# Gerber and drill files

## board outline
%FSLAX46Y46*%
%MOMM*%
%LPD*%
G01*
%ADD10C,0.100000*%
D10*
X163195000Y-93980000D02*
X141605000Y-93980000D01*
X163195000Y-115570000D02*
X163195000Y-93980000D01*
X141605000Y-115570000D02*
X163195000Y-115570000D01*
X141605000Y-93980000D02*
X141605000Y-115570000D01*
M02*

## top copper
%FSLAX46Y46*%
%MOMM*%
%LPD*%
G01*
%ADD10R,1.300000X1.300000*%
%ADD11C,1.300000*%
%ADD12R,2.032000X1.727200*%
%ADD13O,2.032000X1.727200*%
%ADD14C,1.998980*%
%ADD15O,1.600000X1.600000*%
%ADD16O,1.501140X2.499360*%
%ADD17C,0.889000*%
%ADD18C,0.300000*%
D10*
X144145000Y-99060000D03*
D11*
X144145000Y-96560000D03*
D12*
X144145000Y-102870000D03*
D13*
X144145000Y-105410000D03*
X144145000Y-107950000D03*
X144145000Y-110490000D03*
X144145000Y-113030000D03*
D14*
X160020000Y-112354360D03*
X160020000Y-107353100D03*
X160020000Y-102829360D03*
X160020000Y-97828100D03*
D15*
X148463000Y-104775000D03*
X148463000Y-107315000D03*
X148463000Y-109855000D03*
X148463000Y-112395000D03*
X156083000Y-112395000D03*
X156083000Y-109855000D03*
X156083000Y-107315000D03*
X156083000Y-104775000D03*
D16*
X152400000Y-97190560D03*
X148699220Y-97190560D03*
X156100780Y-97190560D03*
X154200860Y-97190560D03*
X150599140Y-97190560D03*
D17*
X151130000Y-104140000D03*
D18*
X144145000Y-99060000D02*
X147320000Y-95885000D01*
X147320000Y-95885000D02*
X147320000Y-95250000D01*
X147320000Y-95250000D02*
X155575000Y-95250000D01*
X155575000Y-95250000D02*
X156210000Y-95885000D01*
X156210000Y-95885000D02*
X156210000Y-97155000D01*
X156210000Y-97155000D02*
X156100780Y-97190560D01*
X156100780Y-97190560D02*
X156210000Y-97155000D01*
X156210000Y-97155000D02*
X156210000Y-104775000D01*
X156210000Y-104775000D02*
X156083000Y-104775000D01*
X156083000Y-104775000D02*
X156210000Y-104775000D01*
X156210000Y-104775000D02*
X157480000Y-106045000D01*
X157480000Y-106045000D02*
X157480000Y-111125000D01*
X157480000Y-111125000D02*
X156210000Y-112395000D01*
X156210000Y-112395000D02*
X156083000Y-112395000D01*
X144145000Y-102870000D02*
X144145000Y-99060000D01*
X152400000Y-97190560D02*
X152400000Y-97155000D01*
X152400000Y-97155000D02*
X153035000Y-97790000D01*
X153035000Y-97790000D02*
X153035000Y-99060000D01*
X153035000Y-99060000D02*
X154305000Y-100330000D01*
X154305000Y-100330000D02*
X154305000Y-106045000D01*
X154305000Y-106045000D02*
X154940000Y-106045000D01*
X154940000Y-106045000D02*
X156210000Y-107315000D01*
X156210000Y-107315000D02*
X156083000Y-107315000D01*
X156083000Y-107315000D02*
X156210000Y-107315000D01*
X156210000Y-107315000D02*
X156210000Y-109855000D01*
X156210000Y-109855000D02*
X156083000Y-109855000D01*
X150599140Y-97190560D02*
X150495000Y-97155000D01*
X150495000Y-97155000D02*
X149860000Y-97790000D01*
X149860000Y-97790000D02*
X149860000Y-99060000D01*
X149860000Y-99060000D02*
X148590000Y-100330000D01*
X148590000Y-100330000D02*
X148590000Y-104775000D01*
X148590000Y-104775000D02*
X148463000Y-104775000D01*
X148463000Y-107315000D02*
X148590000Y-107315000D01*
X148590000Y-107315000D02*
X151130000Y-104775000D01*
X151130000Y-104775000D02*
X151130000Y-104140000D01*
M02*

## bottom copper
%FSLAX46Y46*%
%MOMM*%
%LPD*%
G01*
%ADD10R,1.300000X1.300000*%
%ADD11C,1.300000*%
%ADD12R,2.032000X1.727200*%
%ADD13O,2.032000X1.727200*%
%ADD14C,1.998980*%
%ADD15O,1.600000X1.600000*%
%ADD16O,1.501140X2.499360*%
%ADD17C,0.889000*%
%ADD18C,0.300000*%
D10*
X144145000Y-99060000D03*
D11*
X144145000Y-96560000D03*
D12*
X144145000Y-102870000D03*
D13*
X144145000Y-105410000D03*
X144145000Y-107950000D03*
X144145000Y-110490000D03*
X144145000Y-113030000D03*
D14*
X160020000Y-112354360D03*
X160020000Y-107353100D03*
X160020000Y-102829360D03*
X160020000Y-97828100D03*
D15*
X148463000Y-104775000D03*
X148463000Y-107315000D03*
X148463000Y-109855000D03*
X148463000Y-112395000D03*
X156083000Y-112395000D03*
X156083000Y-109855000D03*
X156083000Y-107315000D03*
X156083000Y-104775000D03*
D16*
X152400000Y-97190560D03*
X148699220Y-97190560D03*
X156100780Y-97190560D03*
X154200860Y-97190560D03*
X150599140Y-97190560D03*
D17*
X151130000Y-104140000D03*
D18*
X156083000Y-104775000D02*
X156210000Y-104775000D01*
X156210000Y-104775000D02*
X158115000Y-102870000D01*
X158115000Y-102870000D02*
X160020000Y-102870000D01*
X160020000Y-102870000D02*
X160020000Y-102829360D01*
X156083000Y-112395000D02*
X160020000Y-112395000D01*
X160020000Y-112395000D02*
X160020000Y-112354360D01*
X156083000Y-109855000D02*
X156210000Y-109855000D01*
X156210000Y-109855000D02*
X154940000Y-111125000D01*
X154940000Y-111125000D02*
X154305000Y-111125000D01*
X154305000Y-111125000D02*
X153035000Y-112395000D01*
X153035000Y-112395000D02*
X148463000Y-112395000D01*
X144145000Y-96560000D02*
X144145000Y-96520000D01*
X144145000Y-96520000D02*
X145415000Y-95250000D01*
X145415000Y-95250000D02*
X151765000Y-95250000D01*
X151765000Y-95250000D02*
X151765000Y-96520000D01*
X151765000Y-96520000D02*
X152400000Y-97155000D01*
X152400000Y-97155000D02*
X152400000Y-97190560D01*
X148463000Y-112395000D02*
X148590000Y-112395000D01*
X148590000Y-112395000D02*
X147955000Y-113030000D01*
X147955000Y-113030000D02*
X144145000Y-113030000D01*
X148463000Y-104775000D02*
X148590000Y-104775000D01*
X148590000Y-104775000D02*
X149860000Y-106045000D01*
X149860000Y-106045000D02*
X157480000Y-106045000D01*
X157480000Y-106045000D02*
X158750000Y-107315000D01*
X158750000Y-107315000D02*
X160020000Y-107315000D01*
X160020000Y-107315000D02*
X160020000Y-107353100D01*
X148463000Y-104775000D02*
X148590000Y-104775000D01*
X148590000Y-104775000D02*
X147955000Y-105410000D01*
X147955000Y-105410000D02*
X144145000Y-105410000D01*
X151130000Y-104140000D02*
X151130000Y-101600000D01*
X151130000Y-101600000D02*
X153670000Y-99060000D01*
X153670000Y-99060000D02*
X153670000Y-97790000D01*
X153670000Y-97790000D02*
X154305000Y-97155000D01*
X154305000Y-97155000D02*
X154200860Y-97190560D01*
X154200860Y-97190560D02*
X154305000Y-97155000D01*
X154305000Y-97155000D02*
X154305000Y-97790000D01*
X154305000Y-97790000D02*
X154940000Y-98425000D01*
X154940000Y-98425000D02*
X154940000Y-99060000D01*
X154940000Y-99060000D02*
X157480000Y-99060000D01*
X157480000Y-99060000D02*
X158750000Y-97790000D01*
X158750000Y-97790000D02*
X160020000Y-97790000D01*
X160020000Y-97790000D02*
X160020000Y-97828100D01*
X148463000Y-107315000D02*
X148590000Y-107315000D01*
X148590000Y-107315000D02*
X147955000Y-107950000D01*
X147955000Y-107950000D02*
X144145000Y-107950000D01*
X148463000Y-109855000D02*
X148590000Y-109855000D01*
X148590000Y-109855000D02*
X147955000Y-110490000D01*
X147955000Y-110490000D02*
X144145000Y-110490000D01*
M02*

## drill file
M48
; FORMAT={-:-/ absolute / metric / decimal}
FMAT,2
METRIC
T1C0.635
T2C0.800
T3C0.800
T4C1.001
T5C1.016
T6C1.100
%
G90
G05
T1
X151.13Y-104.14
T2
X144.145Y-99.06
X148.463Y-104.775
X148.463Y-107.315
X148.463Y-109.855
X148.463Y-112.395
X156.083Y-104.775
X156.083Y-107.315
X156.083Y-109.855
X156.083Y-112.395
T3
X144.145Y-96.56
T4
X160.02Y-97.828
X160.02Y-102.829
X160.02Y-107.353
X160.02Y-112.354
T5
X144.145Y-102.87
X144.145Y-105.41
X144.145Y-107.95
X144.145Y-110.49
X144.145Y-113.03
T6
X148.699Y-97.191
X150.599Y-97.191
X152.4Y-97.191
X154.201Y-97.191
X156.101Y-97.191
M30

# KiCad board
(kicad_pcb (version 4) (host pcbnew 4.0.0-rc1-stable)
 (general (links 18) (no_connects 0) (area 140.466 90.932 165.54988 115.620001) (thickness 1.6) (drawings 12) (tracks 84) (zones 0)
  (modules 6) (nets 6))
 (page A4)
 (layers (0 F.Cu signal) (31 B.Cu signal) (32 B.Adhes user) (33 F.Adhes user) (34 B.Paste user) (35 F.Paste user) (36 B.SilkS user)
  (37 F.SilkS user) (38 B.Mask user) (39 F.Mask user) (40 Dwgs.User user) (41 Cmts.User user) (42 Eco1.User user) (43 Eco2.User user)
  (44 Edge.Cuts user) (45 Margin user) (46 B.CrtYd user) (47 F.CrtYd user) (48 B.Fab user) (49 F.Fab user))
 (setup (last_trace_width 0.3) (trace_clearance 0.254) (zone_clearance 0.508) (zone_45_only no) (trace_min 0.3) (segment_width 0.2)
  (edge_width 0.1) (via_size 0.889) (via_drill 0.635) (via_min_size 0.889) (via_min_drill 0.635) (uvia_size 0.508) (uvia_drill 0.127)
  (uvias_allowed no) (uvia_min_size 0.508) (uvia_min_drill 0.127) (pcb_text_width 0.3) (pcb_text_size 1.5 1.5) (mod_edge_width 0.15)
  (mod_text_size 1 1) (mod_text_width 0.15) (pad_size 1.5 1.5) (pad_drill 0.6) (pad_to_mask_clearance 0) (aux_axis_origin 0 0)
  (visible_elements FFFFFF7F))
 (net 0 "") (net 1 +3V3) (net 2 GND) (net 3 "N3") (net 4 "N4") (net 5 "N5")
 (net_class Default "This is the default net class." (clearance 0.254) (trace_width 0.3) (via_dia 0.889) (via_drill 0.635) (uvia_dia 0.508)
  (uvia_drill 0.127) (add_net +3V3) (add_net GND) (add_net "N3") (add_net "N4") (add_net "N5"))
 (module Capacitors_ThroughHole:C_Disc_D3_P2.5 (layer F.Cu) (at 144.145 99.06 90)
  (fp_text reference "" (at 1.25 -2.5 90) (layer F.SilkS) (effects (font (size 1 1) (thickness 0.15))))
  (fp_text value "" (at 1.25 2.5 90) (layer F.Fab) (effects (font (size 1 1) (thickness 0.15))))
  (pad 1 thru_hole rect (at 0 0 90) (size 1.3 1.3) (drill 0.8) (layers *.Cu *.Mask F.SilkS) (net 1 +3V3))
  (pad 2 thru_hole circle (at 2.5 0 90) (size 1.3 1.3) (drill 0.8001) (layers *.Cu *.Mask F.SilkS) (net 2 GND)))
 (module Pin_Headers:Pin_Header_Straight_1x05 (layer F.Cu) (at 144.145 102.87)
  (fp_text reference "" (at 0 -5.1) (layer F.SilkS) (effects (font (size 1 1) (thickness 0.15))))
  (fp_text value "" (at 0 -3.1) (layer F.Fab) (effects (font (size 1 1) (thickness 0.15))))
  (pad 1 thru_hole rect (at 0 0) (size 2.032 1.7272) (drill 1.016) (layers *.Cu *.Mask F.SilkS) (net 1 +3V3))
  (pad 2 thru_hole oval (at 0 2.54) (size 2.032 1.7272) (drill 1.016) (layers *.Cu *.Mask F.SilkS) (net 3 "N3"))
  (pad 3 thru_hole oval (at 0 5.08) (size 2.032 1.7272) (drill 1.016) (layers *.Cu *.Mask F.SilkS) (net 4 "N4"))
  (pad 4 thru_hole oval (at 0 7.62) (size 2.032 1.7272) (drill 1.016) (layers *.Cu *.Mask F.SilkS) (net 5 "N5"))
  (pad 5 thru_hole oval (at 0 10.16) (size 2.032 1.7272) (drill 1.016) (layers *.Cu *.Mask F.SilkS) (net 2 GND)))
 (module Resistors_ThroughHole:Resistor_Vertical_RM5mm (layer F.Cu) (at 160.02 109.855 90)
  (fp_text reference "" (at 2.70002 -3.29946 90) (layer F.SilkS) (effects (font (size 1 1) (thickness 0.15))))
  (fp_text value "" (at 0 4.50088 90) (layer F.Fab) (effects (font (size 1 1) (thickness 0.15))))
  (pad 1 thru_hole circle (at -2.49936 0 90) (size 1.99898 1.99898) (drill 1.00076) (layers *.Cu *.SilkS *.Mask) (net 1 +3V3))
  (pad 2 thru_hole circle (at 2.5019 0 90) (size 1.99898 1.99898) (drill 1.00076) (layers *.Cu *.SilkS *.Mask) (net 3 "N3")))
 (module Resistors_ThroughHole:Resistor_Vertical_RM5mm (layer F.Cu) (at 160.02 100.33 90)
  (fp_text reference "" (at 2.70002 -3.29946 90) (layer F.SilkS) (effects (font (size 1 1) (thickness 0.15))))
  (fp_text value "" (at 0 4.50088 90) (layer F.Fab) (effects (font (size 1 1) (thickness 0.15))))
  (pad 1 thru_hole circle (at -2.49936 0 90) (size 1.99898 1.99898) (drill 1.00076) (layers *.Cu *.SilkS *.Mask) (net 1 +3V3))
  (pad 2 thru_hole circle (at 2.5019 0 90) (size 1.99898 1.99898) (drill 1.00076) (layers *.Cu *.SilkS *.Mask) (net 4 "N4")))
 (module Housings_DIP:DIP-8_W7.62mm (layer F.Cu) (at 148.463 104.775)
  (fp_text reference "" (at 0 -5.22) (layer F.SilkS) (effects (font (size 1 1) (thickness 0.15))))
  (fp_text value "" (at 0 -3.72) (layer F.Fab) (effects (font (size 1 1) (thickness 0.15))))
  (pad 1 thru_hole oval (at 0 0) (size 1.6 1.6) (drill 0.8) (layers *.Cu *.Mask F.SilkS) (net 3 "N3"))
  (pad 2 thru_hole oval (at 0 2.54) (size 1.6 1.6) (drill 0.8) (layers *.Cu *.Mask F.SilkS) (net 4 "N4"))
  (pad 3 thru_hole oval (at 0 5.08) (size 1.6 1.6) (drill 0.8) (layers *.Cu *.Mask F.SilkS) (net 5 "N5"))
  (pad 4 thru_hole oval (at 0 7.62) (size 1.6 1.6) (drill 0.8) (layers *.Cu *.Mask F.SilkS) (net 2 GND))
  (pad 5 thru_hole oval (at 7.62 7.62) (size 1.6 1.6) (drill 0.8) (layers *.Cu *.Mask F.SilkS) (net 1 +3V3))
  (pad 6 thru_hole oval (at 7.62 5.08) (size 1.6 1.6) (drill 0.8) (layers *.Cu *.Mask F.SilkS) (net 2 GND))
  (pad 7 thru_hole oval (at 7.62 2.54) (size 1.6 1.6) (drill 0.8) (layers *.Cu *.Mask F.SilkS) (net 2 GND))
  (pad 8 thru_hole oval (at 7.62 0) (size 1.6 1.6) (drill 0.8) (layers *.Cu *.Mask F.SilkS) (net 1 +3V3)))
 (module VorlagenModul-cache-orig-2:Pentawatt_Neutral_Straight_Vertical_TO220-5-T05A (layer F.Cu) (at 152.4 97.79)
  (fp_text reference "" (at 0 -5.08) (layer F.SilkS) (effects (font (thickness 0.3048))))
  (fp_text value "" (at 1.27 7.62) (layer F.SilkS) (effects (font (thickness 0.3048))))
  (pad 3 thru_hole oval (at 0 -0.59944 90) (size 2.49936 1.50114) (drill 1.09982) (layers *.Cu *.Mask F.SilkS) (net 2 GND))
  (pad 1 thru_hole oval (at -3.70078 -0.59944 90) (size 2.49936 1.50114) (drill 1.09982) (layers *.Cu *.Mask F.SilkS))
  (pad 5 thru_hole oval (at 3.70078 -0.59944 90) (size 2.49936 1.50114) (drill 1.09982) (layers *.Cu *.Mask F.SilkS) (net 1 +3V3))
  (pad 4 thru_hole oval (at 1.80086 -0.59944 90) (size 2.49936 1.50114) (drill 1.09982) (layers *.Cu *.Mask F.SilkS) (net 4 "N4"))
  (pad 2 thru_hole oval (at -1.80086 -0.59944 90) (size 2.49936 1.50114) (drill 1.09982) (layers *.Cu *.Mask F.SilkS) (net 3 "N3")))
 (gr_line (start 163.195 93.98) (end 141.605 93.98) (angle 90) (layer Edge.Cuts) (width 0.1))
 (gr_line (start 163.195 115.57) (end 163.195 93.98) (angle 90) (layer Edge.Cuts) (width 0.1))
 (gr_line (start 141.605 115.57) (end 163.195 115.57) (angle 90) (layer Edge.Cuts) (width 0.1))
 (gr_line (start 141.605 93.98) (end 141.605 115.57) (angle 90) (layer Edge.Cuts) (width 0.1))
 (segment (start 144.145 99.06) (end 147.32 95.885) (width 0.3) (layer F.Cu) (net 1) (status 80000))
 (segment (start 147.32 95.885) (end 147.32 95.25) (width 0.3) (layer F.Cu) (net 1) (status 80000))
 (segment (start 147.32 95.25) (end 155.575 95.25) (width 0.3) (layer F.Cu) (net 1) (status 80000))
 (segment (start 155.575 95.25) (end 156.21 95.885) (width 0.3) (layer F.Cu) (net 1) (status 80000))
 (segment (start 156.21 95.885) (end 156.21 97.155) (width 0.3) (layer F.Cu) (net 1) (status 80000))
 (segment (start 156.21 97.155) (end 156.10078 97.19056) (width 0.3) (layer F.Cu) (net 1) (status 80000))
 (segment (start 156.083 104.775) (end 156.21 104.775) (width 0.3) (layer B.Cu) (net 1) (status 80000))
 (segment (start 156.21 104.775) (end 158.115 102.87) (width 0.3) (layer B.Cu) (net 1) (status 80000))
 (segment (start 158.115 102.87) (end 160.02 102.87) (width 0.3) (layer B.Cu) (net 1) (status 80000))
 (segment (start 160.02 102.87) (end 160.02 102.82936) (width 0.3) (layer B.Cu) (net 1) (status 80000))
 (segment (start 156.10078 97.19056) (end 156.21 97.155) (width 0.3) (layer F.Cu) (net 1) (status 80000))
 (segment (start 156.21 97.155) (end 156.21 104.775) (width 0.3) (layer F.Cu) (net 1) (status 80000))
 (segment (start 156.21 104.775) (end 156.083 104.775) (width 0.3) (layer F.Cu) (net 1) (status 80000))
 (segment (start 156.083 104.775) (end 156.21 104.775) (width 0.3) (layer F.Cu) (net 1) (status 80000))
 (segment (start 156.21 104.775) (end 157.48 106.045) (width 0.3) (layer F.Cu) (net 1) (status 80000))
 (segment (start 157.48 106.045) (end 157.48 111.125) (width 0.3) (layer F.Cu) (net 1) (status 80000))
 (segment (start 157.48 111.125) (end 156.21 112.395) (width 0.3) (layer F.Cu) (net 1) (status 80000))
 (segment (start 156.21 112.395) (end 156.083 112.395) (width 0.3) (layer F.Cu) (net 1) (status 80000))
 (segment (start 156.083 112.395) (end 160.02 112.395) (width 0.3) (layer B.Cu) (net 1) (status 80000))
 (segment (start 160.02 112.395) (end 160.02 112.35436) (width 0.3) (layer B.Cu) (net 1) (status 80000))
 (segment (start 144.145 102.87) (end 144.145 99.06) (width 0.3) (layer F.Cu) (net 1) (status 80000))
 (segment (start 152.4 97.19056) (end 152.4 97.155) (width 0.3) (layer F.Cu) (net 2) (status 80000))
 (segment (start 152.4 97.155) (end 153.035 97.79) (width 0.3) (layer F.Cu) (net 2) (status 80000))
 (segment (start 153.035 97.79) (end 153.035 99.06) (width 0.3) (layer F.Cu) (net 2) (status 80000))
 (segment (start 153.035 99.06) (end 154.305 100.33) (width 0.3) (layer F.Cu) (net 2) (status 80000))
 (segment (start 154.305 100.33) (end 154.305 106.045) (width 0.3) (layer F.Cu) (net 2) (status 80000))
 (segment (start 154.305 106.045) (end 154.94 106.045) (width 0.3) (layer F.Cu) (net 2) (status 80000))
 (segment (start 154.94 106.045) (end 156.21 107.315) (width 0.3) (layer F.Cu) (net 2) (status 80000))
 (segment (start 156.21 107.315) (end 156.083 107.315) (width 0.3) (layer F.Cu) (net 2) (status 80000))
 (segment (start 156.083 109.855) (end 156.21 109.855) (width 0.3) (layer B.Cu) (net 2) (status 80000))
 (segment (start 156.21 109.855) (end 154.94 111.125) (width 0.3) (layer B.Cu) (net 2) (status 80000))
 (segment (start 154.94 111.125) (end 154.305 111.125) (width 0.3) (layer B.Cu) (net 2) (status 80000))
 (segment (start 154.305 111.125) (end 153.035 112.395) (width 0.3) (layer B.Cu) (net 2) (status 80000))
 (segment (start 153.035 112.395) (end 148.463 112.395) (width 0.3) (layer B.Cu) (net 2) (status 80000))
 (segment (start 144.145 96.56) (end 144.145 96.52) (width 0.3) (layer B.Cu) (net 2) (status 80000))
 (segment (start 144.145 96.52) (end 145.415 95.25) (width 0.3) (layer B.Cu) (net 2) (status 80000))
 (segment (start 145.415 95.25) (end 151.765 95.25) (width 0.3) (layer B.Cu) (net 2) (status 80000))
 (segment (start 151.765 95.25) (end 151.765 96.52) (width 0.3) (layer B.Cu) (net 2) (status 80000))
 (segment (start 151.765 96.52) (end 152.4 97.155) (width 0.3) (layer B.Cu) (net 2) (status 80000))
 (segment (start 152.4 97.155) (end 152.4 97.19056) (width 0.3) (layer B.Cu) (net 2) (status 80000))
 (segment (start 148.463 112.395) (end 148.59 112.395) (width 0.3) (layer B.Cu) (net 2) (status 80000))
 (segment (start 148.59 112.395) (end 147.955 113.03) (width 0.3) (layer B.Cu) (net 2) (status 80000))
 (segment (start 147.955 113.03) (end 144.145 113.03) (width 0.3) (layer B.Cu) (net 2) (status 80000))
 (segment (start 156.083 107.315) (end 156.21 107.315) (width 0.3) (layer F.Cu) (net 2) (status 80000))
 (segment (start 156.21 107.315) (end 156.21 109.855) (width 0.3) (layer F.Cu) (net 2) (status 80000))
 (segment (start 156.21 109.855) (end 156.083 109.855) (width 0.3) (layer F.Cu) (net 2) (status 80000))
 (segment (start 148.463 104.775) (end 148.59 104.775) (width 0.3) (layer B.Cu) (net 3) (status 80000))
 (segment (start 148.59 104.775) (end 149.86 106.045) (width 0.3) (layer B.Cu) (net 3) (status 80000))
 (segment (start 149.86 106.045) (end 157.48 106.045) (width 0.3) (layer B.Cu) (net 3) (status 80000))
 (segment (start 157.48 106.045) (end 158.75 107.315) (width 0.3) (layer B.Cu) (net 3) (status 80000))
 (segment (start 158.75 107.315) (end 160.02 107.315) (width 0.3) (layer B.Cu) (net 3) (status 80000))
 (segment (start 160.02 107.315) (end 160.02 107.3531) (width 0.3) (layer B.Cu) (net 3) (status 80000))
 (segment (start 150.59914 97.19056) (end 150.495 97.155) (width 0.3) (layer F.Cu) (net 3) (status 80000))
 (segment (start 150.495 97.155) (end 149.86 97.79) (width 0.3) (layer F.Cu) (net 3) (status 80000))
 (segment (start 149.86 97.79) (end 149.86 99.06) (width 0.3) (layer F.Cu) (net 3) (status 80000))
 (segment (start 149.86 99.06) (end 148.59 100.33) (width 0.3) (layer F.Cu) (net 3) (status 80000))
 (segment (start 148.59 100.33) (end 148.59 104.775) (width 0.3) (layer F.Cu) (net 3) (status 80000))
 (segment (start 148.59 104.775) (end 148.463 104.775) (width 0.3) (layer F.Cu) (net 3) (status 80000))
 (segment (start 148.463 104.775) (end 148.59 104.775) (width 0.3) (layer B.Cu) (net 3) (status 80000))
 (segment (start 148.59 104.775) (end 147.955 105.41) (width 0.3) (layer B.Cu) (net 3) (status 80000))
 (segment (start 147.955 105.41) (end 144.145 105.41) (width 0.3) (layer B.Cu) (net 3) (status 80000))
 (segment (start 148.463 107.315) (end 148.59 107.315) (width 0.3) (layer F.Cu) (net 4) (status 80000))
 (segment (start 148.59 107.315) (end 151.13 104.775) (width 0.3) (layer F.Cu) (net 4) (status 80000))
 (segment (start 151.13 104.775) (end 151.13 104.14) (width 0.3) (layer F.Cu) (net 4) (status 80000))
 (via (at 151.13 104.14) (size 0.889) (layers F.Cu B.Cu) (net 4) (status 80000))
 (segment (start 151.13 104.14) (end 151.13 101.6) (width 0.3) (layer B.Cu) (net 4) (status 80000))
 (segment (start 151.13 101.6) (end 153.67 99.06) (width 0.3) (layer B.Cu) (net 4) (status 80000))
 (segment (start 153.67 99.06) (end 153.67 97.79) (width 0.3) (layer B.Cu) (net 4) (status 80000))
 (segment (start 153.67 97.79) (end 154.305 97.155) (width 0.3) (layer B.Cu) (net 4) (status 80000))
 (segment (start 154.305 97.155) (end 154.20086 97.19056) (width 0.3) (layer B.Cu) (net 4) (status 80000))
 (segment (start 154.20086 97.19056) (end 154.305 97.155) (width 0.3) (layer B.Cu) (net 4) (status 80000))
 (segment (start 154.305 97.155) (end 154.305 97.79) (width 0.3) (layer B.Cu) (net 4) (status 80000))
 (segment (start 154.305 97.79) (end 154.94 98.425) (width 0.3) (layer B.Cu) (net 4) (status 80000))
 (segment (start 154.94 98.425) (end 154.94 99.06) (width 0.3) (layer B.Cu) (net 4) (status 80000))
 (segment (start 154.94 99.06) (end 157.48 99.06) (width 0.3) (layer B.Cu) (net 4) (status 80000))
 (segment (start 157.48 99.06) (end 158.75 97.79) (width 0.3) (layer B.Cu) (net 4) (status 80000))
 (segment (start 158.75 97.79) (end 160.02 97.79) (width 0.3) (layer B.Cu) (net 4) (status 80000))
 (segment (start 160.02 97.79) (end 160.02 97.8281) (width 0.3) (layer B.Cu) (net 4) (status 80000))
 (segment (start 148.463 107.315) (end 148.59 107.315) (width 0.3) (layer B.Cu) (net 4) (status 80000))
 (segment (start 148.59 107.315) (end 147.955 107.95) (width 0.3) (layer B.Cu) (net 4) (status 80000))
 (segment (start 147.955 107.95) (end 144.145 107.95) (width 0.3) (layer B.Cu) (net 4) (status 80000))
 (segment (start 148.463 109.855) (end 148.59 109.855) (width 0.3) (layer B.Cu) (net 5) (status 80000))
 (segment (start 148.59 109.855) (end 147.955 110.49) (width 0.3) (layer B.Cu) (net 5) (status 80000))
 (segment (start 147.955 110.49) (end 144.145 110.49) (width 0.3) (layer B.Cu) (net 5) (status 80000)))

